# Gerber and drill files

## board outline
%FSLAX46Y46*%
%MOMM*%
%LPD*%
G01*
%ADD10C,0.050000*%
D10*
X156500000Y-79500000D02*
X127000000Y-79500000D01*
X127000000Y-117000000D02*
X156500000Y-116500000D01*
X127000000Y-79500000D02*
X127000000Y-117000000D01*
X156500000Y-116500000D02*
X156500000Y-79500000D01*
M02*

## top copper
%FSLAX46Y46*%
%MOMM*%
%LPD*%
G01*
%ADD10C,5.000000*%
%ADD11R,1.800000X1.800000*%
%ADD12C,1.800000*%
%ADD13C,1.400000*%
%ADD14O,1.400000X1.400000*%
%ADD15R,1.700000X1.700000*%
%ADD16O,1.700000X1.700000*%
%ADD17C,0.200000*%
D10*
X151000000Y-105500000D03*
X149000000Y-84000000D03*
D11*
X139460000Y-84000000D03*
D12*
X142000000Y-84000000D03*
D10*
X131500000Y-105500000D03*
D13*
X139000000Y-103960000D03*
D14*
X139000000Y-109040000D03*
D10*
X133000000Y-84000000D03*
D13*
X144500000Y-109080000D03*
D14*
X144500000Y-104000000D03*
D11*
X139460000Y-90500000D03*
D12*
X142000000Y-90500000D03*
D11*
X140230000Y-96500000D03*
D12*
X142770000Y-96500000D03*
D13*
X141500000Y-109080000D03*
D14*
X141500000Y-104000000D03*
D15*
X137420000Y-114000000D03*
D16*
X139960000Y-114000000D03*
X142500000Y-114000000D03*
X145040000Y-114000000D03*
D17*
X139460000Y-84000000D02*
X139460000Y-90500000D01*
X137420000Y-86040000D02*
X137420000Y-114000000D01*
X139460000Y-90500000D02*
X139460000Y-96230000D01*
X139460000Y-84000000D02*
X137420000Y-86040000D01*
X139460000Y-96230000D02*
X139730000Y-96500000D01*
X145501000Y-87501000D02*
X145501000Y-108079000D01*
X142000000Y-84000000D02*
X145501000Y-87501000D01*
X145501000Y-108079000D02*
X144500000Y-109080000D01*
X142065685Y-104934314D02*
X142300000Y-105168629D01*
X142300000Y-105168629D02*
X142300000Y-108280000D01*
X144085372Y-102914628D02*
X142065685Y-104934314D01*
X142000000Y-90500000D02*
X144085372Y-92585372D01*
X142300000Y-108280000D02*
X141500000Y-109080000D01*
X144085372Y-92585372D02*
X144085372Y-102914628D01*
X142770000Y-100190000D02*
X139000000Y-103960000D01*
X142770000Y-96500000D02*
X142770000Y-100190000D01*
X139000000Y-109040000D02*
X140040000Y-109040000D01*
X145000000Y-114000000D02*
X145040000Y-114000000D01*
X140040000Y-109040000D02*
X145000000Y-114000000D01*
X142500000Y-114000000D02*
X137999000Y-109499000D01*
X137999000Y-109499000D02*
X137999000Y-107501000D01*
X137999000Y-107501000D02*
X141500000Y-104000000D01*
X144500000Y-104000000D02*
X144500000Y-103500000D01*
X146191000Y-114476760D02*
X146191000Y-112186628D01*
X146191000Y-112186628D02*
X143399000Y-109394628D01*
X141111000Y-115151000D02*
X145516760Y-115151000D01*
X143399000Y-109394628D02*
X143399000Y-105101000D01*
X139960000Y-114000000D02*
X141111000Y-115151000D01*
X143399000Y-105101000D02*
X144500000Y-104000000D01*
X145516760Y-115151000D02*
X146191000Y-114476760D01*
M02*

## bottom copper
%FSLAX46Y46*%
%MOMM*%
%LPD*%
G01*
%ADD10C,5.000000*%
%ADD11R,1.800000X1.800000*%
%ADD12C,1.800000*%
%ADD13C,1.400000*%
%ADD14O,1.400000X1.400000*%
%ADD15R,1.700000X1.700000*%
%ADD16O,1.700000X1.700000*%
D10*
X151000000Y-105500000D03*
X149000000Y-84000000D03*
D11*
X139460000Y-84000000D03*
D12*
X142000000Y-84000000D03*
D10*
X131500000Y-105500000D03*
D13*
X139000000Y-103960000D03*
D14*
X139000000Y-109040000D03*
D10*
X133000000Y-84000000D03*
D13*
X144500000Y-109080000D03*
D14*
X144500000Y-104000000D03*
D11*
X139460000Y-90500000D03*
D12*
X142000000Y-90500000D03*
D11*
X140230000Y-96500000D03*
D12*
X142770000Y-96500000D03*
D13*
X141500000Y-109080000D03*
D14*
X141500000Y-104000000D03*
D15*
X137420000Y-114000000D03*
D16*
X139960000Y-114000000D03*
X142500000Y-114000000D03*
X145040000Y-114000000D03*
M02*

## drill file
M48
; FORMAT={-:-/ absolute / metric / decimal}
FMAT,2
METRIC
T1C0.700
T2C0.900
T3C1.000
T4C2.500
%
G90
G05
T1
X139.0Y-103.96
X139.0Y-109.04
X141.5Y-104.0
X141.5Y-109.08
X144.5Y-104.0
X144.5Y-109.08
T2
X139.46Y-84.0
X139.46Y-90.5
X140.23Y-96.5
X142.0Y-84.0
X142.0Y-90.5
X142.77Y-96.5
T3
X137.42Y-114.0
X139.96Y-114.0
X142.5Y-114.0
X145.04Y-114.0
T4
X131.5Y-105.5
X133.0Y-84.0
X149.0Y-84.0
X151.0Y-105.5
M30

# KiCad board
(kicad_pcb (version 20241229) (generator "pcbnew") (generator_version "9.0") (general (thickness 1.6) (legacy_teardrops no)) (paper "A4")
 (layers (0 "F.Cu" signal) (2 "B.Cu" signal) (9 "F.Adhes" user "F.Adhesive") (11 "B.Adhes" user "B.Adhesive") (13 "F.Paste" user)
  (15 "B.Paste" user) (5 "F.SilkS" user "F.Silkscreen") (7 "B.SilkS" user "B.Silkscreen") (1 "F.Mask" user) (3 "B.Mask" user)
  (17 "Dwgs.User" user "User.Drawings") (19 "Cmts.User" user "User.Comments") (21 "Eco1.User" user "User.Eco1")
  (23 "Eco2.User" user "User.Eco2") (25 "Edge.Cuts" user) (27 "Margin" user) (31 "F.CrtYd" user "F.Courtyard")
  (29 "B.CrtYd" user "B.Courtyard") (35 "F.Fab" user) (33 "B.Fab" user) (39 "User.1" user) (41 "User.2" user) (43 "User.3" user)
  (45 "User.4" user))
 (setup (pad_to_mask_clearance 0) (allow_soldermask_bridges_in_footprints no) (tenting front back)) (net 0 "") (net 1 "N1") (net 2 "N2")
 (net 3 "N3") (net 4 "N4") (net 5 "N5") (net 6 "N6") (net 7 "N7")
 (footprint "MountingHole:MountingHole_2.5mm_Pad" (layer "F.Cu") (at 151 105.5)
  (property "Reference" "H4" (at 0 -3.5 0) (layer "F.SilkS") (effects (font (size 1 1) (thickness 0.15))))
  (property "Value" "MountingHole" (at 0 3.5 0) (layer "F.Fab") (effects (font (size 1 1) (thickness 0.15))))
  (pad "1" thru_hole circle (at 0 0) (size 5 5) (drill 2.5) (layers "*.Cu" "*.Mask") (remove_unused_layers no)))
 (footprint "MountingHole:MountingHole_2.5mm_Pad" (layer "F.Cu") (at 149 84)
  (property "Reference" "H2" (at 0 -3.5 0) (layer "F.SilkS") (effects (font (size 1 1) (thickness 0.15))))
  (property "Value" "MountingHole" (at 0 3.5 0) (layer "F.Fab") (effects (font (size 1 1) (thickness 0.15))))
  (pad "1" thru_hole circle (at 0 0) (size 5 5) (drill 2.5) (layers "*.Cu" "*.Mask") (remove_unused_layers no)))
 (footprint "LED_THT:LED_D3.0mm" (layer "F.Cu") (at 139.46 84)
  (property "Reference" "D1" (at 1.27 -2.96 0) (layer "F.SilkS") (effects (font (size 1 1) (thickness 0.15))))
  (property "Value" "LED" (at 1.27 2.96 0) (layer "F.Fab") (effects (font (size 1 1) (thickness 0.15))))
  (pad "1" thru_hole rect (at 0 0) (size 1.8 1.8) (drill 0.9) (layers "*.Cu" "*.Mask") (remove_unused_layers no) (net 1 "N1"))
  (pad "2" thru_hole circle (at 2.54 0) (size 1.8 1.8) (drill 0.9) (layers "*.Cu" "*.Mask") (remove_unused_layers no) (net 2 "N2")))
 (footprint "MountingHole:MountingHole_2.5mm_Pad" (layer "F.Cu") (at 131.5 105.5)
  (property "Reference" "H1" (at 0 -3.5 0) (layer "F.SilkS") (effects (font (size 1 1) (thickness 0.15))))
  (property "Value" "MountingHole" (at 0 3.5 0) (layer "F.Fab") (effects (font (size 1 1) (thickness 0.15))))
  (pad "1" thru_hole circle (at 0 0) (size 5 5) (drill 2.5) (layers "*.Cu" "*.Mask") (remove_unused_layers no)))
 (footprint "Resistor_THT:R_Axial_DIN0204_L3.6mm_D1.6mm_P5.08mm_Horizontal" (layer "F.Cu") (at 139 103.96 -90)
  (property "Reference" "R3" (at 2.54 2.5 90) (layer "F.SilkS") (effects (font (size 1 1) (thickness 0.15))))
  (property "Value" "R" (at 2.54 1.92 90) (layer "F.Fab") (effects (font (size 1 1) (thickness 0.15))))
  (pad "1" thru_hole circle (at 0 0 270) (size 1.4 1.4) (drill 0.7) (layers "*.Cu" "*.Mask") (remove_unused_layers no) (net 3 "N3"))
  (pad "2" thru_hole oval (at 5.08 0 270) (size 1.4 1.4) (drill 0.7) (layers "*.Cu" "*.Mask") (remove_unused_layers no) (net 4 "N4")))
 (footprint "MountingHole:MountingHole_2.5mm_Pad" (layer "F.Cu") (at 133 84)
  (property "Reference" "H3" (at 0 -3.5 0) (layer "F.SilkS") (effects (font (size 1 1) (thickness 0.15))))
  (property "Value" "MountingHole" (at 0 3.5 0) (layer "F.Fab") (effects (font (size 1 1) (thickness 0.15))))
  (pad "1" thru_hole circle (at 0 0) (size 5 5) (drill 2.5) (layers "*.Cu" "*.Mask") (remove_unused_layers no)))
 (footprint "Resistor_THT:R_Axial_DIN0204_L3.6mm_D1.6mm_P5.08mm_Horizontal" (layer "F.Cu") (at 144.5 109.08 90)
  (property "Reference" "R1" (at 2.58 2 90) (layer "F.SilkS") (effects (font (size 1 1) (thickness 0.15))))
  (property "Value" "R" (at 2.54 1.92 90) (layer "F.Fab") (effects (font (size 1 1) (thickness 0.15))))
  (pad "1" thru_hole circle (at 0 0 90) (size 1.4 1.4) (drill 0.7) (layers "*.Cu" "*.Mask") (remove_unused_layers no) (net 2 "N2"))
  (pad "2" thru_hole oval (at 5.08 0 90) (size 1.4 1.4) (drill 0.7) (layers "*.Cu" "*.Mask") (remove_unused_layers no) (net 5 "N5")))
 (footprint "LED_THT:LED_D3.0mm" (layer "F.Cu") (at 139.46 90.5)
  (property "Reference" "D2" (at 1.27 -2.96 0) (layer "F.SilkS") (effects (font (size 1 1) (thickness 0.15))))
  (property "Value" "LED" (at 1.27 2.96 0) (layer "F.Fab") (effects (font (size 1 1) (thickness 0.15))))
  (pad "1" thru_hole rect (at 0 0) (size 1.8 1.8) (drill 0.9) (layers "*.Cu" "*.Mask") (remove_unused_layers no) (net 1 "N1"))
  (pad "2" thru_hole circle (at 2.54 0) (size 1.8 1.8) (drill 0.9) (layers "*.Cu" "*.Mask") (remove_unused_layers no) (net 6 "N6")))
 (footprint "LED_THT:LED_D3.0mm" (layer "F.Cu") (at 140.23 96.5)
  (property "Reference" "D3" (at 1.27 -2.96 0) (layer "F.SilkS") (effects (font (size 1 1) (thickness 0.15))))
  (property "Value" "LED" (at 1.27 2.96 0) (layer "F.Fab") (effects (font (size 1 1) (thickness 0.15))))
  (pad "1" thru_hole rect (at 0 0) (size 1.8 1.8) (drill 0.9) (layers "*.Cu" "*.Mask") (remove_unused_layers no) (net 1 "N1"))
  (pad "2" thru_hole circle (at 2.54 0) (size 1.8 1.8) (drill 0.9) (layers "*.Cu" "*.Mask") (remove_unused_layers no) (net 3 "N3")))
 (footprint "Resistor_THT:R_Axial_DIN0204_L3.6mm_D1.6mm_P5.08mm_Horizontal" (layer "F.Cu") (at 141.5 109.08 90)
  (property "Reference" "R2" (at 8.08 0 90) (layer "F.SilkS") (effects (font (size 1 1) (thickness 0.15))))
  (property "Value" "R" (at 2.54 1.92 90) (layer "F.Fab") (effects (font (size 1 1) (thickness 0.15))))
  (pad "1" thru_hole circle (at 0 0 90) (size 1.4 1.4) (drill 0.7) (layers "*.Cu" "*.Mask") (remove_unused_layers no) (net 6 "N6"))
  (pad "2" thru_hole oval (at 5.08 0 90) (size 1.4 1.4) (drill 0.7) (layers "*.Cu" "*.Mask") (remove_unused_layers no) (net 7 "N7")))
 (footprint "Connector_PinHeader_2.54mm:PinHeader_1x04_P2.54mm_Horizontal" (layer "B.Cu") (at 137.42 114 -90)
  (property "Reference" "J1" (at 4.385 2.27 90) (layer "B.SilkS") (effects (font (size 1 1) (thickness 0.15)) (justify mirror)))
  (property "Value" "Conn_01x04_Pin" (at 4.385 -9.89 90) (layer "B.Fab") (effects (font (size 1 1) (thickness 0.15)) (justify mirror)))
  (pad "1" thru_hole rect (at 0 0 270) (size 1.7 1.7) (drill 1) (layers "*.Cu" "*.Mask") (remove_unused_layers no) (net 1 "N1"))
  (pad "2" thru_hole oval (at 0 -2.54 270) (size 1.7 1.7) (drill 1) (layers "*.Cu" "*.Mask") (remove_unused_layers no) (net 5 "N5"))
  (pad "3" thru_hole oval (at 0 -5.08 270) (size 1.7 1.7) (drill 1) (layers "*.Cu" "*.Mask") (remove_unused_layers no) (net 7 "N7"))
  (pad "4" thru_hole oval (at 0 -7.62 270) (size 1.7 1.7) (drill 1) (layers "*.Cu" "*.Mask") (remove_unused_layers no) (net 4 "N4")))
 (gr_line (start 156.5 79.5) (end 127 79.5) (stroke (width 0.05) (type default)) (layer "Edge.Cuts"))
 (gr_line (start 127 117) (end 156.5 116.5) (stroke (width 0.05) (type default)) (layer "Edge.Cuts"))
 (gr_line (start 127 79.5) (end 127 117) (stroke (width 0.05) (type default)) (layer "Edge.Cuts"))
 (gr_line (start 156.5 116.5) (end 156.5 79.5) (stroke (width 0.05) (type default)) (layer "Edge.Cuts"))
 (segment (start 139.46 84) (end 139.46 90.5) (width 0.2) (layer "F.Cu") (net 1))
 (segment (start 137.42 86.04) (end 137.42 114) (width 0.2) (layer "F.Cu") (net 1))
 (segment (start 139.46 90.5) (end 139.46 96.23) (width 0.2) (layer "F.Cu") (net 1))
 (segment (start 139.46 84) (end 137.42 86.04) (width 0.2) (layer "F.Cu") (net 1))
 (segment (start 139.46 96.23) (end 139.73 96.5) (width 0.2) (layer "F.Cu") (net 1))
 (segment (start 145.501 87.501) (end 145.501 108.079) (width 0.2) (layer "F.Cu") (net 2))
 (segment (start 142 84) (end 145.501 87.501) (width 0.2) (layer "F.Cu") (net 2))
 (segment (start 145.501 108.079) (end 144.5 109.08) (width 0.2) (layer "F.Cu") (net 2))
 (segment (start 142.065685 104.934314) (end 142.3 105.168629) (width 0.2) (layer "F.Cu") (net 6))
 (segment (start 142.3 105.168629) (end 142.3 108.28) (width 0.2) (layer "F.Cu") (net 6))
 (segment (start 144.085372 102.914628) (end 142.065685 104.934314) (width 0.2) (layer "F.Cu") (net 6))
 (segment (start 142 90.5) (end 144.085372 92.585372) (width 0.2) (layer "F.Cu") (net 6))
 (segment (start 142.3 108.28) (end 141.5 109.08) (width 0.2) (layer "F.Cu") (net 6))
 (segment (start 144.085372 92.585372) (end 144.085372 102.914628) (width 0.2) (layer "F.Cu") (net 6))
 (segment (start 142.77 100.19) (end 139 103.96) (width 0.2) (layer "F.Cu") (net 3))
 (segment (start 142.77 96.5) (end 142.77 100.19) (width 0.2) (layer "F.Cu") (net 3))
 (segment (start 139 109.04) (end 140.04 109.04) (width 0.2) (layer "F.Cu") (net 4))
 (segment (start 145 114) (end 145.04 114) (width 0.2) (layer "F.Cu") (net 4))
 (segment (start 140.04 109.04) (end 145 114) (width 0.2) (layer "F.Cu") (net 4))
 (segment (start 142.5 114) (end 137.999 109.499) (width 0.2) (layer "F.Cu") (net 7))
 (segment (start 137.999 109.499) (end 137.999 107.501) (width 0.2) (layer "F.Cu") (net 7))
 (segment (start 137.999 107.501) (end 141.5 104) (width 0.2) (layer "F.Cu") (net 7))
 (segment (start 144.5 104) (end 144.5 103.5) (width 0.2) (layer "F.Cu") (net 5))
 (segment (start 146.191 114.47676) (end 146.191 112.186628) (width 0.2) (layer "F.Cu") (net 5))
 (segment (start 146.191 112.186628) (end 143.399 109.394628) (width 0.2) (layer "F.Cu") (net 5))
 (segment (start 141.111 115.151) (end 145.51676 115.151) (width 0.2) (layer "F.Cu") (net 5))
 (segment (start 143.399 109.394628) (end 143.399 105.101) (width 0.2) (layer "F.Cu") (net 5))
 (segment (start 139.96 114) (end 141.111 115.151) (width 0.2) (layer "F.Cu") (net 5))
 (segment (start 143.399 105.101) (end 144.5 104) (width 0.2) (layer "F.Cu") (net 5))
 (segment (start 145.51676 115.151) (end 146.191 114.47676) (width 0.2) (layer "F.Cu") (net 5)))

